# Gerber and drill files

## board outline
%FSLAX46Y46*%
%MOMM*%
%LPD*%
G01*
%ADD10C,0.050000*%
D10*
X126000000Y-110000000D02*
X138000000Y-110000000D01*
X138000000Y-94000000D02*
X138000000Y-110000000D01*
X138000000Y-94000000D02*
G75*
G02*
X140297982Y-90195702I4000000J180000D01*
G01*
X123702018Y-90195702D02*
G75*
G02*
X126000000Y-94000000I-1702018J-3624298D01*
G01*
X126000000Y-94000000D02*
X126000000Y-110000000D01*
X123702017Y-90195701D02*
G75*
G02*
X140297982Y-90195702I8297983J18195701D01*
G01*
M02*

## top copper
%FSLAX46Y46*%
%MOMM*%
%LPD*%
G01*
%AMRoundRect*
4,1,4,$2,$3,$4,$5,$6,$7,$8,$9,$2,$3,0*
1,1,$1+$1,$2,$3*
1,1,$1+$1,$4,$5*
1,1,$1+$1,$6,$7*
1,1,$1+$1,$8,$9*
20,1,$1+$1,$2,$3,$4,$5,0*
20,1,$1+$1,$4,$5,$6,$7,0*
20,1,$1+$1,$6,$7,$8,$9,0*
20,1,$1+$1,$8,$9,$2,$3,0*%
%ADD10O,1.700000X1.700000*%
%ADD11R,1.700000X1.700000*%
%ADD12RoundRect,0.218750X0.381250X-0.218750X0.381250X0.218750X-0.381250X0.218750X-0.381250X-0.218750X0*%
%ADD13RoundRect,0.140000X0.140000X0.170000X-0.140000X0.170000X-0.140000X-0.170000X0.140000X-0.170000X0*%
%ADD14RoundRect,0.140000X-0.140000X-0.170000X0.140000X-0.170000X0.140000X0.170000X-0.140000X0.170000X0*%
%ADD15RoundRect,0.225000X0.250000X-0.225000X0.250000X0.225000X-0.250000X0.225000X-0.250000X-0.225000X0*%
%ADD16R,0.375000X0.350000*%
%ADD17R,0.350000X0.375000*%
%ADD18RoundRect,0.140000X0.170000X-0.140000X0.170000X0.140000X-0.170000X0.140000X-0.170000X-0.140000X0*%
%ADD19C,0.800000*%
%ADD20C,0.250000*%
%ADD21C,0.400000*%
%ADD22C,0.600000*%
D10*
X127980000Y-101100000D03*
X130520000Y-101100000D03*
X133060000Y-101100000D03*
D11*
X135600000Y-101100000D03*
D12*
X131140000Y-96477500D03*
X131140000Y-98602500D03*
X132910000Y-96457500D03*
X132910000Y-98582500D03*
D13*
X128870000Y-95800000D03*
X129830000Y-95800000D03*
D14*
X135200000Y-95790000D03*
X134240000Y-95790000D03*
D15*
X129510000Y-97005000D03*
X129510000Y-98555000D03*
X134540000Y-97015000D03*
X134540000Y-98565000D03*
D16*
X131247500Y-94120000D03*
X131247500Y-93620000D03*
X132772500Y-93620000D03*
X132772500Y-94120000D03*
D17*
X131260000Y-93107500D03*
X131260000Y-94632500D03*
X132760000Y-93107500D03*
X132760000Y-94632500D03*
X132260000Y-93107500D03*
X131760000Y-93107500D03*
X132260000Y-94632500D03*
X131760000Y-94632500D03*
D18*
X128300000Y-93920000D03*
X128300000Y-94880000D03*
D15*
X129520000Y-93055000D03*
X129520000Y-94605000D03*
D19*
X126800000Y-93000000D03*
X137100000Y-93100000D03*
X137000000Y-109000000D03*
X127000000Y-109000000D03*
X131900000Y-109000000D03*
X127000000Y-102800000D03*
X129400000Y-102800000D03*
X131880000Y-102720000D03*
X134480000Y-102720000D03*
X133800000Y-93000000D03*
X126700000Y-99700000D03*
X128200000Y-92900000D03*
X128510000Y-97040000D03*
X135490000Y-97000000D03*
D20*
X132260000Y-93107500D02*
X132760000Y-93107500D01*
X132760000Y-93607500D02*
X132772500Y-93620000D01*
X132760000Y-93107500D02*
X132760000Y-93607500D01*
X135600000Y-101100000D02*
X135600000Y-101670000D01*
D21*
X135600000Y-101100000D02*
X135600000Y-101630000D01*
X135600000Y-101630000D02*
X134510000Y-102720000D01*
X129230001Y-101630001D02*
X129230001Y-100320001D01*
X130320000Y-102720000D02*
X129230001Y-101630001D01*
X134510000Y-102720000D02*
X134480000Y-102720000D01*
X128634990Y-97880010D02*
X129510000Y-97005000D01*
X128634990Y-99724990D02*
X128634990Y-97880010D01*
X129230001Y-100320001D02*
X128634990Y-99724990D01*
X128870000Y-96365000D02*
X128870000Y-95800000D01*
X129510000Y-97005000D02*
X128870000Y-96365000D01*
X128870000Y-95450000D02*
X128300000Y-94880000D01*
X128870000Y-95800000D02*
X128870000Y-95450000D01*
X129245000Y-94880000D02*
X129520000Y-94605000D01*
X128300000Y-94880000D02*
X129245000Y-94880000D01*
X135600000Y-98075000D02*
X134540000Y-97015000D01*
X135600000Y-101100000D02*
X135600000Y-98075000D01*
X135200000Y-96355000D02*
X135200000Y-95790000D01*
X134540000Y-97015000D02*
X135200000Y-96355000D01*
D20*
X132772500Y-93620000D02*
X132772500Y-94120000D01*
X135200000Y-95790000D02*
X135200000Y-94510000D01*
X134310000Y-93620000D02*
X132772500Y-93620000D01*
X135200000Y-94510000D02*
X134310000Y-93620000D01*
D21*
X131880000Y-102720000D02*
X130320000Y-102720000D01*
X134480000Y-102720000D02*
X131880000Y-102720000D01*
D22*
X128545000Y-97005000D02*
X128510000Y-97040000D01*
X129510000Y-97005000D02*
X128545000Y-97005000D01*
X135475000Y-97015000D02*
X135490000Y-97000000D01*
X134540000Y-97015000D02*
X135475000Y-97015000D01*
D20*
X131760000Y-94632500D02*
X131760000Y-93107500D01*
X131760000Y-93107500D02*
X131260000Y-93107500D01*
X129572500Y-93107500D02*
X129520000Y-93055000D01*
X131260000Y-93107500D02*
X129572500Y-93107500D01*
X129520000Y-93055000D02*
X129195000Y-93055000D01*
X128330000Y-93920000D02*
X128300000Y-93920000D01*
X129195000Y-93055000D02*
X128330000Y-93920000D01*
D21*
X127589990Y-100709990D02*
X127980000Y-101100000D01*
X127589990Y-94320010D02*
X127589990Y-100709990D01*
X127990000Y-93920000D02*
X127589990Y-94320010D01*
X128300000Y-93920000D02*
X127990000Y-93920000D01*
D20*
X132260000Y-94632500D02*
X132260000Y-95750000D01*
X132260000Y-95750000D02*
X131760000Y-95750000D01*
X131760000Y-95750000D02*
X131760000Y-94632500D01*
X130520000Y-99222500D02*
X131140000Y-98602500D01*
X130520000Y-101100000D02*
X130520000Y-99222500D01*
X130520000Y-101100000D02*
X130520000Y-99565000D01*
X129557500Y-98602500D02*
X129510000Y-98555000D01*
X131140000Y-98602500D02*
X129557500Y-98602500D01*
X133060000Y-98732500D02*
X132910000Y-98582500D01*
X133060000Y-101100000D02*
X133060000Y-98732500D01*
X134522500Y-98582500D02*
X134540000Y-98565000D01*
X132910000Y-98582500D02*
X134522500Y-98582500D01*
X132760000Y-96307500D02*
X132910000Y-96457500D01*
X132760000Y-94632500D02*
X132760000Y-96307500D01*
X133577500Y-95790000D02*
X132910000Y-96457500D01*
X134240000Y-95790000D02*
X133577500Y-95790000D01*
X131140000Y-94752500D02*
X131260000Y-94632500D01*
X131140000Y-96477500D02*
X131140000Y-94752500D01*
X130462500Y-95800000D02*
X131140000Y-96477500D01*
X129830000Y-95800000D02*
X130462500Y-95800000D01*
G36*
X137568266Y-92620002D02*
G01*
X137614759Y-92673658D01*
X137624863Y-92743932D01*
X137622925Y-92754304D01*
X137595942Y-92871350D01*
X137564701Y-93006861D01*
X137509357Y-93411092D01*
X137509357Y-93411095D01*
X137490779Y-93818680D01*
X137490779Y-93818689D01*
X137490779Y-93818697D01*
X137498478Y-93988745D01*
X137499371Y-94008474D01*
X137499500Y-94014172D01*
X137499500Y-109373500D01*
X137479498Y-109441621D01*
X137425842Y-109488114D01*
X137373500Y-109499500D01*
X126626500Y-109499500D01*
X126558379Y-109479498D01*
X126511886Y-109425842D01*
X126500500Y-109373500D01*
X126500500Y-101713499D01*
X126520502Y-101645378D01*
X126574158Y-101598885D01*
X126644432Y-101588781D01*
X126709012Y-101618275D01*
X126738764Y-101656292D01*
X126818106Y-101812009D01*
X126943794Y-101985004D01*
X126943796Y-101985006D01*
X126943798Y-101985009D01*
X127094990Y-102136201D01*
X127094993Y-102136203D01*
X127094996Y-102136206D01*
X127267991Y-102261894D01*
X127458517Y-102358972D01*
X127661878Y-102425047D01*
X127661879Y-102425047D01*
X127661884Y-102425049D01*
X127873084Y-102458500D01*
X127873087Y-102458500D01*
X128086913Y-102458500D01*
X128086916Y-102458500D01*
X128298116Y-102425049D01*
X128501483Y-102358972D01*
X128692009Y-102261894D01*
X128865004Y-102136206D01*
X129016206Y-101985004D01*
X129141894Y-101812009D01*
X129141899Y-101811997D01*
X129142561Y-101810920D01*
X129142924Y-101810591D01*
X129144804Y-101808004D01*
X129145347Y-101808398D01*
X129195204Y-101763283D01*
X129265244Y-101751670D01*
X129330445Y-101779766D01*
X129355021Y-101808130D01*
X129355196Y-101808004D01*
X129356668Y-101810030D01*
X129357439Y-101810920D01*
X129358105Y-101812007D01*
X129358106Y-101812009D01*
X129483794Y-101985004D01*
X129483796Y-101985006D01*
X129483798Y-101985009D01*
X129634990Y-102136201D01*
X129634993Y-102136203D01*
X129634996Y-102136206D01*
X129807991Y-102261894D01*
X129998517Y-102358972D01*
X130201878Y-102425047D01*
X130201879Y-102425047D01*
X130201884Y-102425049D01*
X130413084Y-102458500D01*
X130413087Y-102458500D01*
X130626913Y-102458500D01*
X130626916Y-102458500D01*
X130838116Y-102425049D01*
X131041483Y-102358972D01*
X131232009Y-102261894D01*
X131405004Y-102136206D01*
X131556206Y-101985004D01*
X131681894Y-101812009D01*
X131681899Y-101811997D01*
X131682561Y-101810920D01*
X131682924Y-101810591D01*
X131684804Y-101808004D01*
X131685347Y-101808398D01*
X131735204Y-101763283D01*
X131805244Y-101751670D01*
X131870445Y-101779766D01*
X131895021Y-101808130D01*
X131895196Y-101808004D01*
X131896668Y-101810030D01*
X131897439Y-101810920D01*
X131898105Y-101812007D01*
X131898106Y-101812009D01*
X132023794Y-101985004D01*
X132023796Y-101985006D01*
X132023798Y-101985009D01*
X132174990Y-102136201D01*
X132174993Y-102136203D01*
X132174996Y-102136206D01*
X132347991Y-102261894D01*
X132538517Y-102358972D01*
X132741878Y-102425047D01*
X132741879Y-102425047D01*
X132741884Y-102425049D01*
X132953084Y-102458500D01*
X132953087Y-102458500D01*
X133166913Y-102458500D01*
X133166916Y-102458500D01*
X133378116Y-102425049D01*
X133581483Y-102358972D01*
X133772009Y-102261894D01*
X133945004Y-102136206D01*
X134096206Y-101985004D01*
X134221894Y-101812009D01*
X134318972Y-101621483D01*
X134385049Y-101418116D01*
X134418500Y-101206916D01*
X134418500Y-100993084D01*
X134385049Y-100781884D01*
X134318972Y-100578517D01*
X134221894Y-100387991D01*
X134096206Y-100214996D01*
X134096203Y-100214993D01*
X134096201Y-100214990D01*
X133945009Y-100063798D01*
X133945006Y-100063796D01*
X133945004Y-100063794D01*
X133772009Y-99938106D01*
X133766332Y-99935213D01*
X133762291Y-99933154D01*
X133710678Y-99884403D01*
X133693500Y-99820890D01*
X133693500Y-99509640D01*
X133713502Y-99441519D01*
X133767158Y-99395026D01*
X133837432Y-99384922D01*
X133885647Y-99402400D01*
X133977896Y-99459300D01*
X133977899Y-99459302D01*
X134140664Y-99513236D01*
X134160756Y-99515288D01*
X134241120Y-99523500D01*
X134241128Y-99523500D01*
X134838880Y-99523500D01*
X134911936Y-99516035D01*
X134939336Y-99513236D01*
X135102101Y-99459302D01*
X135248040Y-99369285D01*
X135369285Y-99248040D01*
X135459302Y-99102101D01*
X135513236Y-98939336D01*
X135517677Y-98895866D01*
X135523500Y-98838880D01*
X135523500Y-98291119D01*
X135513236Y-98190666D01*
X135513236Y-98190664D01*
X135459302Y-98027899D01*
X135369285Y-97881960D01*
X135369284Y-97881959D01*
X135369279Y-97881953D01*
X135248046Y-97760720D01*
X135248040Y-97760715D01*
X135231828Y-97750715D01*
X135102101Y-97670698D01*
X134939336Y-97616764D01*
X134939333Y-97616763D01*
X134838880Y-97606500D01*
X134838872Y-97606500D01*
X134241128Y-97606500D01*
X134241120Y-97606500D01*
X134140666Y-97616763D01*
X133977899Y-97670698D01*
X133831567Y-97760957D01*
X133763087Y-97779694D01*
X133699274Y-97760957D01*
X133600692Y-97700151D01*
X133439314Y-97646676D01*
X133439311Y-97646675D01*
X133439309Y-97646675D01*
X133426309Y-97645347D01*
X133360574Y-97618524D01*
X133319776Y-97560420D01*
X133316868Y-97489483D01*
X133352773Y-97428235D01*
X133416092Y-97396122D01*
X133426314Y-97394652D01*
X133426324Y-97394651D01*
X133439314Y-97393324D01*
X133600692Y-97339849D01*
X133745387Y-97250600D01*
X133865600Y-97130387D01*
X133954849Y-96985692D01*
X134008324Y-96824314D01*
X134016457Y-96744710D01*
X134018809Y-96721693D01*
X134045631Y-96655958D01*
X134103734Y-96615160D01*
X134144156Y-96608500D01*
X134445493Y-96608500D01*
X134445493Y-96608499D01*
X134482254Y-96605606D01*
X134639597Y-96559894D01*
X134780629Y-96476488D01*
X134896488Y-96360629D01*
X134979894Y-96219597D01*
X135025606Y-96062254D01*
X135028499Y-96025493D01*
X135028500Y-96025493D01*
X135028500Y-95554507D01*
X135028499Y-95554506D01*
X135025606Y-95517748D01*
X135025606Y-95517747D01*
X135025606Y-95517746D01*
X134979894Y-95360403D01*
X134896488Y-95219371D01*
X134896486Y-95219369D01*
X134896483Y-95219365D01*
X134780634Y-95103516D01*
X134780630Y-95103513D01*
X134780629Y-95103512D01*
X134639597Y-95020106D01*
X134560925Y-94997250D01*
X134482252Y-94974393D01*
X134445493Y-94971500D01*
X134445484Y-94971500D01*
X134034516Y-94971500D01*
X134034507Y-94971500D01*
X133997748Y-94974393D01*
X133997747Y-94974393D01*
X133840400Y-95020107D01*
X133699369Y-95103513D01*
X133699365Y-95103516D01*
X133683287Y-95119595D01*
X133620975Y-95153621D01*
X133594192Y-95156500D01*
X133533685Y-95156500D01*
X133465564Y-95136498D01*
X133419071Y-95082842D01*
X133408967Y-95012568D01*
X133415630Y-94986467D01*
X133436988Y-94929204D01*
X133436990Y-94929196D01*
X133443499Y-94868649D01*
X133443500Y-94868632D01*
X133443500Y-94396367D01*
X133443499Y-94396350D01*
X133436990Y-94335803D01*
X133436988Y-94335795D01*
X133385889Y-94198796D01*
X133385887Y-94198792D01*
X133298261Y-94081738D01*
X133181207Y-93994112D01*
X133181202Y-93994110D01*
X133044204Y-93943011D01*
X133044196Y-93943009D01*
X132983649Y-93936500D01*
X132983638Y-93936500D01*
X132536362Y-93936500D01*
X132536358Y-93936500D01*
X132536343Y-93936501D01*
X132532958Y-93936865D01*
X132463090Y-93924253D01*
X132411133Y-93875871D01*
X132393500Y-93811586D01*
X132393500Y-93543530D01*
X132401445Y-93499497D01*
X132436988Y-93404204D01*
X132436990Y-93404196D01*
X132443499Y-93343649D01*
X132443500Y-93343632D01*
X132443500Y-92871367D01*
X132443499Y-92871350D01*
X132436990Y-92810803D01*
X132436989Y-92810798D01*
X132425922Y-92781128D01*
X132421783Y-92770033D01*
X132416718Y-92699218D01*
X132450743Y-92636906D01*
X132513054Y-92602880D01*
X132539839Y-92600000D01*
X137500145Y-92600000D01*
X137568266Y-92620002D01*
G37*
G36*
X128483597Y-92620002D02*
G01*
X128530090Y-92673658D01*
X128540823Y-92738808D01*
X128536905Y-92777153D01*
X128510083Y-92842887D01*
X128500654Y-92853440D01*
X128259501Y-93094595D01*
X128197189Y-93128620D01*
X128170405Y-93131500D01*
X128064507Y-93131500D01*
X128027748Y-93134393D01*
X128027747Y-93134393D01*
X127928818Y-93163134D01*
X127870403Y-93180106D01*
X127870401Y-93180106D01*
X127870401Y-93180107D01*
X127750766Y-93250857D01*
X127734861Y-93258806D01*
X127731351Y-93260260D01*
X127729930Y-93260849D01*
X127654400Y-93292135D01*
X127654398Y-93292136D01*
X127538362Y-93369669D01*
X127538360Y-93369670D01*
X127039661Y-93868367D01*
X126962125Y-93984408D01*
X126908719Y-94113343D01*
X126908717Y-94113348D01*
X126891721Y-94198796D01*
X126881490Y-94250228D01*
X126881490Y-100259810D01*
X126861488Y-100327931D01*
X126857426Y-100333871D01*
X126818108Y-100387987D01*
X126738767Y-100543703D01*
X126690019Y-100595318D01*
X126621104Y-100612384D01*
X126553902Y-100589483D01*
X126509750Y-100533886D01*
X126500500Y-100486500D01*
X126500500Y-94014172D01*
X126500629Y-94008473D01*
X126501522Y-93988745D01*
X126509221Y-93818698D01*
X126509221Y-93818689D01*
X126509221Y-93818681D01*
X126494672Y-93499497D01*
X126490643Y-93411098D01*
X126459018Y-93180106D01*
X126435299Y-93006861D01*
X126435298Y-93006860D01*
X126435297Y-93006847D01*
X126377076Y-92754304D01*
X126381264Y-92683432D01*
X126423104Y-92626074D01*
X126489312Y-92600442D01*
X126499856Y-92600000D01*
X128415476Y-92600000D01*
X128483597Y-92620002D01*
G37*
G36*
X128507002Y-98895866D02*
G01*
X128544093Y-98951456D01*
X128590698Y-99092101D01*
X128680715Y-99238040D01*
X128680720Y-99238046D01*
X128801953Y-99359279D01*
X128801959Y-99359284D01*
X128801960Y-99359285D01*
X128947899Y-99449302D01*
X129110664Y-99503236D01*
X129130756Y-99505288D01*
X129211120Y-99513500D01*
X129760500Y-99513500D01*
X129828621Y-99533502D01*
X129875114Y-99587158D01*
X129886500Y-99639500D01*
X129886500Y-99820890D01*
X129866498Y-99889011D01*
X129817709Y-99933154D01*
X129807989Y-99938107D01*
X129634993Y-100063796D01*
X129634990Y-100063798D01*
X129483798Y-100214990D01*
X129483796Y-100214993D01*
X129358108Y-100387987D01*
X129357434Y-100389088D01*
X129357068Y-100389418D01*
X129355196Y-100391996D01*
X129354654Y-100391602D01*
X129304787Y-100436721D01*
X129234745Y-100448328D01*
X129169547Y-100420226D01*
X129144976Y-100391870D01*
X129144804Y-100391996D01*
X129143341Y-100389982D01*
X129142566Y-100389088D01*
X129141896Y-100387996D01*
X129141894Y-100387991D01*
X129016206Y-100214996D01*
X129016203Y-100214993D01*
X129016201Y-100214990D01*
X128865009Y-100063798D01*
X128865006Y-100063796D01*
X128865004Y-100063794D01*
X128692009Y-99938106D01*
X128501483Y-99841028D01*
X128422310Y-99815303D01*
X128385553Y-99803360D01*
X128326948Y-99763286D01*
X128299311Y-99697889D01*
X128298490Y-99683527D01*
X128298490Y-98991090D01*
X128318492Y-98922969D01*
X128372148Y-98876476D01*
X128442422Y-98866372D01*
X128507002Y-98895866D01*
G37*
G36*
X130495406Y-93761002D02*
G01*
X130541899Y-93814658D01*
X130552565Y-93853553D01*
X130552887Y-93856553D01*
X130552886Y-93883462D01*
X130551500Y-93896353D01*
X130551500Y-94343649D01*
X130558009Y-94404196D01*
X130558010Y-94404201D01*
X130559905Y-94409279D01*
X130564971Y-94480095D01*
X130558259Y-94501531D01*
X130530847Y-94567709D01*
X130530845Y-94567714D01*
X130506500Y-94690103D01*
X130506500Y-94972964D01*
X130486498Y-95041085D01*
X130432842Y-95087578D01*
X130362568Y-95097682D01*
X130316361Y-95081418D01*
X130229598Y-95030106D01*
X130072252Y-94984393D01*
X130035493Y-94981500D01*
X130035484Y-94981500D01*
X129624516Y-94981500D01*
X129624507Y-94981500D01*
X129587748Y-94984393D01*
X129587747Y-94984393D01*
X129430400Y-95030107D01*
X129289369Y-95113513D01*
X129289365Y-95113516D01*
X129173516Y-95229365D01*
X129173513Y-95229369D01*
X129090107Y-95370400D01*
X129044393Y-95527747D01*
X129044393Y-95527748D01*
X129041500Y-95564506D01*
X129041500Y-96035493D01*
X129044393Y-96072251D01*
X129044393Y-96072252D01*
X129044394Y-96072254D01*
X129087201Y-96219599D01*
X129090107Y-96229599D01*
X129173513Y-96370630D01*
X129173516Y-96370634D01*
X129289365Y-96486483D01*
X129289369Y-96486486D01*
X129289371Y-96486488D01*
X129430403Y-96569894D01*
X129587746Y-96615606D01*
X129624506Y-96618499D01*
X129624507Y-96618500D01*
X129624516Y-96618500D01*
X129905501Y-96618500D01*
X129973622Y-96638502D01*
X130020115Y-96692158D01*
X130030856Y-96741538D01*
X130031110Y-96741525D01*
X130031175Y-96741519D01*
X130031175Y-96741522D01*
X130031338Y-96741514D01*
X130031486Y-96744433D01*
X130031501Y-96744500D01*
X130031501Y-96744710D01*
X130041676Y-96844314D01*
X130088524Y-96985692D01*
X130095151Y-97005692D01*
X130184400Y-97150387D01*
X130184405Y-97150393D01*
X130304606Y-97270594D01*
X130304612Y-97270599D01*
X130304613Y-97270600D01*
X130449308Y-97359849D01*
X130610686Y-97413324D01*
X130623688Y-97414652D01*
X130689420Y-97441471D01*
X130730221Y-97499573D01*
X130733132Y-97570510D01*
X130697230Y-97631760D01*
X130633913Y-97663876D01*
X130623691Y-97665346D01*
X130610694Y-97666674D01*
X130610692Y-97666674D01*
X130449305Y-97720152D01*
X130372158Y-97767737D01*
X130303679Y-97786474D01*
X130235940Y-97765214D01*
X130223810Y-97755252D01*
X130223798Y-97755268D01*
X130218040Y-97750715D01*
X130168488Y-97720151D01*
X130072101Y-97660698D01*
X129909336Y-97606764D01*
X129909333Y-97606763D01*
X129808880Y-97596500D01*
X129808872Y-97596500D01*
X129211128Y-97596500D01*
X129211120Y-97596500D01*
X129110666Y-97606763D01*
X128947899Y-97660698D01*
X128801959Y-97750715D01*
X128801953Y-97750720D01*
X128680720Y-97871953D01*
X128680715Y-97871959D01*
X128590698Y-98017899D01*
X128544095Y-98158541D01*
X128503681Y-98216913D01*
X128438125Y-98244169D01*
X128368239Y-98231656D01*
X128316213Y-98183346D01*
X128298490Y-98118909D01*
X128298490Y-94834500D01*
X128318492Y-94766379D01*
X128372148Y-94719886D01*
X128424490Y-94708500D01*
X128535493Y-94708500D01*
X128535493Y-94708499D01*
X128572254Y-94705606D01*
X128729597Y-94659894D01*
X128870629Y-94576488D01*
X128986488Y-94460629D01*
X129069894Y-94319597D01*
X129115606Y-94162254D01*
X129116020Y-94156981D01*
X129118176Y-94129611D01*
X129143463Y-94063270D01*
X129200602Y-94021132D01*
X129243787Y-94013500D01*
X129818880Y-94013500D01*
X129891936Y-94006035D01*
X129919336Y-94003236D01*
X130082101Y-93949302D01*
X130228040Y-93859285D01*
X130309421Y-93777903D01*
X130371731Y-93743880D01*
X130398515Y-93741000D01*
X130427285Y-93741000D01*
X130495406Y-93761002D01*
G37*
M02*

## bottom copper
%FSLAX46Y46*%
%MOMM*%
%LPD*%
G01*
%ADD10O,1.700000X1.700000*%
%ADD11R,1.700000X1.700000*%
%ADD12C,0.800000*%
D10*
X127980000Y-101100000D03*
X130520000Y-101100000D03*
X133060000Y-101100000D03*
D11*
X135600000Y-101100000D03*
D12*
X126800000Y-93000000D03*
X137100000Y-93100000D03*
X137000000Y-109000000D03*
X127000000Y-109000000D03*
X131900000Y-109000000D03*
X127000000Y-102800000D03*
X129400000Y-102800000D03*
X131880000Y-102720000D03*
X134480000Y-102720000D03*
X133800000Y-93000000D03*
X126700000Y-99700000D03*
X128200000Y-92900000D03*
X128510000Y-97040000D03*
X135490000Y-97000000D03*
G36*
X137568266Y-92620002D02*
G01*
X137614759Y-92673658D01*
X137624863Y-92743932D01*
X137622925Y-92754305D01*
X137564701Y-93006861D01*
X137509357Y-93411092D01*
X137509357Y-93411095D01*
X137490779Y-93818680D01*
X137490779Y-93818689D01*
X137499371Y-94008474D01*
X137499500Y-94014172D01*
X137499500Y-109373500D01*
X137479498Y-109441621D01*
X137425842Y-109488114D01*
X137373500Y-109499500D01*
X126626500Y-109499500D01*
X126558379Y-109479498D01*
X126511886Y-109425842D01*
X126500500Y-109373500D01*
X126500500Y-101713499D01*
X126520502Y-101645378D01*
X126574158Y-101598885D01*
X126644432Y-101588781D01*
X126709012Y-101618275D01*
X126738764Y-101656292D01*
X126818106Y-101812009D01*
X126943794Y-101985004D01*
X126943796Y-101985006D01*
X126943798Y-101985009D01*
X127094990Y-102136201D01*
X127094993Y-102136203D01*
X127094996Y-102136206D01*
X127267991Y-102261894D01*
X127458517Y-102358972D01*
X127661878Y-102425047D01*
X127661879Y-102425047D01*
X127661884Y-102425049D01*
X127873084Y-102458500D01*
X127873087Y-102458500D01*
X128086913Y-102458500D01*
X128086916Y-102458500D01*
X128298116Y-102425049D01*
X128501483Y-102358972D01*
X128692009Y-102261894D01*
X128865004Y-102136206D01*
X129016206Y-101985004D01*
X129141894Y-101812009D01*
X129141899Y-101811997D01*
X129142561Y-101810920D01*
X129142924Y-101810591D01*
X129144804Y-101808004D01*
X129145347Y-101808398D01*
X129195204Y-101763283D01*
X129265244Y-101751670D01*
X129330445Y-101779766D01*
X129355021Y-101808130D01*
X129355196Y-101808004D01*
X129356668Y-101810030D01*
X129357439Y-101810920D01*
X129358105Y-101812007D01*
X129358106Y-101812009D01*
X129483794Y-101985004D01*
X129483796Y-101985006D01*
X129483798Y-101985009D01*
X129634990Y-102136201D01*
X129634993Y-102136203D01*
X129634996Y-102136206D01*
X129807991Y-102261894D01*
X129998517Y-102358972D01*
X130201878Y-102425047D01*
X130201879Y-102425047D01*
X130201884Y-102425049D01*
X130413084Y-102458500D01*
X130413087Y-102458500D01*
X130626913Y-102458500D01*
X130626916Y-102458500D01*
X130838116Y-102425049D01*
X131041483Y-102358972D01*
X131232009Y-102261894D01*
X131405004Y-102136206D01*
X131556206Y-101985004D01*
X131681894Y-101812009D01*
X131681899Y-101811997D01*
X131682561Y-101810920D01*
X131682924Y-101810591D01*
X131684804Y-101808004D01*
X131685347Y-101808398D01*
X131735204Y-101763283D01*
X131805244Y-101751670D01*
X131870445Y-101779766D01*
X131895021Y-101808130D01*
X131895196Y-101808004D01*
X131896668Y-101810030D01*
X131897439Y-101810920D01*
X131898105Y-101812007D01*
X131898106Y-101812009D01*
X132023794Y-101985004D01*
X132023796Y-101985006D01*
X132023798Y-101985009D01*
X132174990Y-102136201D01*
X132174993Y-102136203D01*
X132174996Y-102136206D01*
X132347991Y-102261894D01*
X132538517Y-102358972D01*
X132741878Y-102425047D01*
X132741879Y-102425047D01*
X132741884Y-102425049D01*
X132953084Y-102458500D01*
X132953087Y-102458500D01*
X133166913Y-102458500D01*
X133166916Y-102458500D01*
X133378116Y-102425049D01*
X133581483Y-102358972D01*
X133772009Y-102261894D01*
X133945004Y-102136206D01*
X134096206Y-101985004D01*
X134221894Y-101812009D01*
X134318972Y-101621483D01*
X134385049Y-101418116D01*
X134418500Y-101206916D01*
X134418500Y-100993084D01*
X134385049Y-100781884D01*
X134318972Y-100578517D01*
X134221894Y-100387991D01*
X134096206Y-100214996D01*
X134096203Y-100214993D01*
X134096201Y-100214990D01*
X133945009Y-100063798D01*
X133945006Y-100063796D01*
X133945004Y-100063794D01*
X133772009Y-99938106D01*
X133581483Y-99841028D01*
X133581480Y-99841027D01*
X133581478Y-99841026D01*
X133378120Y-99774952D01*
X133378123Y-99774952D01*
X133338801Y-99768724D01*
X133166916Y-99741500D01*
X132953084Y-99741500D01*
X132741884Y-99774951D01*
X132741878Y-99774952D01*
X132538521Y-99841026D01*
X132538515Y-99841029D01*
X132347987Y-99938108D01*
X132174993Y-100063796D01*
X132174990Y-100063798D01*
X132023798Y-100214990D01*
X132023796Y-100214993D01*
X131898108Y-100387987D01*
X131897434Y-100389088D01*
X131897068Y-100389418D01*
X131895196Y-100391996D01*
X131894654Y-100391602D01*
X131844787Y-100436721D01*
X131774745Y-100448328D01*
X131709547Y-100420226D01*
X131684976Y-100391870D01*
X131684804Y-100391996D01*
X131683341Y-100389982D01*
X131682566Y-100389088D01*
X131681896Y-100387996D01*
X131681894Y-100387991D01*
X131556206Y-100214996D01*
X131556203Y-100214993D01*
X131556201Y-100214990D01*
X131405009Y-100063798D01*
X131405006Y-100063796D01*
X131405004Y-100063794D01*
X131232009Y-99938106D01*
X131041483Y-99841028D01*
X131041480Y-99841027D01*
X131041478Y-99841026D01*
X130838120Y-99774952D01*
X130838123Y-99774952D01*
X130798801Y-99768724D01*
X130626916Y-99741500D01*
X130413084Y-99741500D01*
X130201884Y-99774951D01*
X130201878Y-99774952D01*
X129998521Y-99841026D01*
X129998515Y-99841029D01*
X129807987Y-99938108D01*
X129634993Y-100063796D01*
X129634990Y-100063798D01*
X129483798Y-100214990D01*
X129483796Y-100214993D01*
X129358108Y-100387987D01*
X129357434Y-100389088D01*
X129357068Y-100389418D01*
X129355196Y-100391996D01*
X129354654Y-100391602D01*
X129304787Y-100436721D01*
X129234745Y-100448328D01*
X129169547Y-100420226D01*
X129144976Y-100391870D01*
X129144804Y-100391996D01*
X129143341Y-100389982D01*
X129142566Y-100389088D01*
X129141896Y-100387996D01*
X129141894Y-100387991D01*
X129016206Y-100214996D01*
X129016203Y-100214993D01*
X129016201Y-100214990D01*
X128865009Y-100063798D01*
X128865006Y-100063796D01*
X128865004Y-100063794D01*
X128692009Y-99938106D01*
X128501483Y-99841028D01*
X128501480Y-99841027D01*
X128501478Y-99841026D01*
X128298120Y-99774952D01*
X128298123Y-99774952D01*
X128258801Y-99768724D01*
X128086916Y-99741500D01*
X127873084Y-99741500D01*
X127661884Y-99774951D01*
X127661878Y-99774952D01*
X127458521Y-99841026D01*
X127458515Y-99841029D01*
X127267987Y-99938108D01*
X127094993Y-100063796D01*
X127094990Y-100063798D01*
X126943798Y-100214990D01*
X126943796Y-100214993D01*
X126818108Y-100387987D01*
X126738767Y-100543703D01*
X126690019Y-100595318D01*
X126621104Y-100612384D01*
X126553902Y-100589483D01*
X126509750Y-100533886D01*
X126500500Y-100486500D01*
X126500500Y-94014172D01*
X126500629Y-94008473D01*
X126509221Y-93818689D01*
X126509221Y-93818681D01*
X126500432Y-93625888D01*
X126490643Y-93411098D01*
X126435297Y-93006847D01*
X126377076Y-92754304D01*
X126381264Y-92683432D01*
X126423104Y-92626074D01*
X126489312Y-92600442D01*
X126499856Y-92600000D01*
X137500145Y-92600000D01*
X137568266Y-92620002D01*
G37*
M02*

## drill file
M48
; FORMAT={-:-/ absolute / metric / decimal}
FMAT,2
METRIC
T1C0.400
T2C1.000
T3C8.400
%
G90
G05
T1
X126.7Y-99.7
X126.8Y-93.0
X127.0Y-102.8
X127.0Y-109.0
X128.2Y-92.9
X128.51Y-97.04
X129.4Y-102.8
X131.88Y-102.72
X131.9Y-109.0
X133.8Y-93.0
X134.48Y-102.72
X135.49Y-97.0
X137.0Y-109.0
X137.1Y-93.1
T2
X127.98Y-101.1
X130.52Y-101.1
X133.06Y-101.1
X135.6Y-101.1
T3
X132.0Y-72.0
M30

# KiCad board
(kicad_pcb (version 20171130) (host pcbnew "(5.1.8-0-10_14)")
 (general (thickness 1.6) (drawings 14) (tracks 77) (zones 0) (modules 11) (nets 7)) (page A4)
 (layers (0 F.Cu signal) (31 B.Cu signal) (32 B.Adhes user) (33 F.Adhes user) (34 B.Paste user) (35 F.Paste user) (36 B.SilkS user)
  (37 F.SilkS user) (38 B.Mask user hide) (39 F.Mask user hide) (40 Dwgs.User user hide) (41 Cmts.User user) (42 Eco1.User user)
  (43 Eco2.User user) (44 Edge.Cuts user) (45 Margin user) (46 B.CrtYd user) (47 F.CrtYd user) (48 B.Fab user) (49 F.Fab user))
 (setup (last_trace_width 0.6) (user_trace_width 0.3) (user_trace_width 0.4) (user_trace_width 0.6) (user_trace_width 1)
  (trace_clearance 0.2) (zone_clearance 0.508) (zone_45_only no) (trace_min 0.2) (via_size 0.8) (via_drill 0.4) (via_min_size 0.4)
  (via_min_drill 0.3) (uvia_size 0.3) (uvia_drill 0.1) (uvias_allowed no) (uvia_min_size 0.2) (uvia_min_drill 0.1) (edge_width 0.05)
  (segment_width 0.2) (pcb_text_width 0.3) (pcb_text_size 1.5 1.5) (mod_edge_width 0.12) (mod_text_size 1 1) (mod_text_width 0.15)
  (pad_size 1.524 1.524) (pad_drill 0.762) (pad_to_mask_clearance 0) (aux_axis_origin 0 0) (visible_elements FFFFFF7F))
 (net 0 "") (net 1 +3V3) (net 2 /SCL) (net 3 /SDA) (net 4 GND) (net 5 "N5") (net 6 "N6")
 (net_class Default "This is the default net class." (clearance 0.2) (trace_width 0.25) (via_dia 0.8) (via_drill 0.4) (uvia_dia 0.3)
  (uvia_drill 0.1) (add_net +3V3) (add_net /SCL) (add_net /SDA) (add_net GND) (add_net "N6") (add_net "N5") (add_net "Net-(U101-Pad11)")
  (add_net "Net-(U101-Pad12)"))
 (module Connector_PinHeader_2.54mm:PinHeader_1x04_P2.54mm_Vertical (layer F.Cu) (at 135.6 101.1 270)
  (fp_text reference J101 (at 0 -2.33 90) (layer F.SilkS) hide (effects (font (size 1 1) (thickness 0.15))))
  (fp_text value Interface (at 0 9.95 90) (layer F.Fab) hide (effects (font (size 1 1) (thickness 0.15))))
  (pad 4 thru_hole oval (at 0 7.62 270) (size 1.7 1.7) (drill 1) (layers *.Cu *.Mask) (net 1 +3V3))
  (pad 3 thru_hole oval (at 0 5.08 270) (size 1.7 1.7) (drill 1) (layers *.Cu *.Mask) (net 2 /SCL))
  (pad 2 thru_hole oval (at 0 2.54 270) (size 1.7 1.7) (drill 1) (layers *.Cu *.Mask) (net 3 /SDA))
  (pad 1 thru_hole rect (at 0 0 270) (size 1.7 1.7) (drill 1) (layers *.Cu *.Mask) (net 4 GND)))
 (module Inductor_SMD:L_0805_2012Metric (layer F.Cu) (at 131.14 97.54 90)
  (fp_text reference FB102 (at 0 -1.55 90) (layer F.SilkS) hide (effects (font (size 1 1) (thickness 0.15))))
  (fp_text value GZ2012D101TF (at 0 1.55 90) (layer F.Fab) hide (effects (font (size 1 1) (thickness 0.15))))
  (pad 2 smd roundrect (at 1.0625 0 90) (size 0.875 1.2) (layers F.Cu F.Paste F.Mask) (roundrect_rratio 0.25) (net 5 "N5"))
  (pad 1 smd roundrect (at -1.0625 0 90) (size 0.875 1.2) (layers F.Cu F.Paste F.Mask) (roundrect_rratio 0.25) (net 2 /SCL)))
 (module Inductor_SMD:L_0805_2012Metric (layer F.Cu) (at 132.91 97.52 90)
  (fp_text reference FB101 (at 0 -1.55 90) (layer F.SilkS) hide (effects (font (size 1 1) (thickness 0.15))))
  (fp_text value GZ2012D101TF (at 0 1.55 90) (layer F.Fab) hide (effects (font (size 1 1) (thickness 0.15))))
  (pad 2 smd roundrect (at 1.0625 0 90) (size 0.875 1.2) (layers F.Cu F.Paste F.Mask) (roundrect_rratio 0.25) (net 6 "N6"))
  (pad 1 smd roundrect (at -1.0625 0 90) (size 0.875 1.2) (layers F.Cu F.Paste F.Mask) (roundrect_rratio 0.25) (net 3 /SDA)))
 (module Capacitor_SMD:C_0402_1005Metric (layer F.Cu) (at 129.35 95.8 180)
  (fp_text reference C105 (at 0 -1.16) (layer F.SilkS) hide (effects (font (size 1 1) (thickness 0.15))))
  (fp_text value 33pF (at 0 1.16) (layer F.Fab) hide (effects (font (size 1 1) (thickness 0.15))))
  (pad 2 smd roundrect (at 0.48 0 180) (size 0.56 0.62) (layers F.Cu F.Paste F.Mask) (roundrect_rratio 0.25) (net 4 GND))
  (pad 1 smd roundrect (at -0.48 0 180) (size 0.56 0.62) (layers F.Cu F.Paste F.Mask) (roundrect_rratio 0.25) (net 5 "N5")))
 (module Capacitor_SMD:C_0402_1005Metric (layer F.Cu) (at 134.72 95.79)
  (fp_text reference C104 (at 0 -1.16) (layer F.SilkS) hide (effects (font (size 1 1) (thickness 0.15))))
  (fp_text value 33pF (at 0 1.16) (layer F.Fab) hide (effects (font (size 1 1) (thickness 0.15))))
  (pad 2 smd roundrect (at 0.48 0) (size 0.56 0.62) (layers F.Cu F.Paste F.Mask) (roundrect_rratio 0.25) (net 4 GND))
  (pad 1 smd roundrect (at -0.48 0) (size 0.56 0.62) (layers F.Cu F.Paste F.Mask) (roundrect_rratio 0.25) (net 6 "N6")))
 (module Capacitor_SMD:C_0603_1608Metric (layer F.Cu) (at 129.51 97.78 90)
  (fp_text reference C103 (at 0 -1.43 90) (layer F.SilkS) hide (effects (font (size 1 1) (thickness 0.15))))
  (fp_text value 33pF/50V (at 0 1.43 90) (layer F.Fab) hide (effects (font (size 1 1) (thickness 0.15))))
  (pad 2 smd roundrect (at 0.775 0 90) (size 0.9 0.95) (layers F.Cu F.Paste F.Mask) (roundrect_rratio 0.25) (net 4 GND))
  (pad 1 smd roundrect (at -0.775 0 90) (size 0.9 0.95) (layers F.Cu F.Paste F.Mask) (roundrect_rratio 0.25) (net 2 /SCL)))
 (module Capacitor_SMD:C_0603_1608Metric (layer F.Cu) (at 134.54 97.79 90)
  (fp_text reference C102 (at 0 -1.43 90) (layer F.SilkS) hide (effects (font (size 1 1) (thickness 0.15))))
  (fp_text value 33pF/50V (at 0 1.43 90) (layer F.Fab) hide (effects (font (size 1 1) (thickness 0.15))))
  (pad 2 smd roundrect (at 0.775 0 90) (size 0.9 0.95) (layers F.Cu F.Paste F.Mask) (roundrect_rratio 0.25) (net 4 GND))
  (pad 1 smd roundrect (at -0.775 0 90) (size 0.9 0.95) (layers F.Cu F.Paste F.Mask) (roundrect_rratio 0.25) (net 3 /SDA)))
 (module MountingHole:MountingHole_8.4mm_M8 (layer F.Cu) (at 132 72)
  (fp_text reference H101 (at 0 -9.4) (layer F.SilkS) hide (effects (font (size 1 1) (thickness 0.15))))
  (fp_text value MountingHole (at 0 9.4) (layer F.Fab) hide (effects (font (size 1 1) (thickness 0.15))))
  (pad 1 np_thru_hole circle (at 0 0) (size 8.4 8.4) (drill 8.4) (layers *.Cu *.Mask)))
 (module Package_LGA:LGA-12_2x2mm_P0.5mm (layer F.Cu) (at 132.01 93.87 90)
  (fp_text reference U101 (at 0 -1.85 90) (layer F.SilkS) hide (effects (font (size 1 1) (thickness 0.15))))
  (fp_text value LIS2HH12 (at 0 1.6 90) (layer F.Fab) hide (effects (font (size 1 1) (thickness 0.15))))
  (pad 12 smd rect (at -0.25 -0.7625 180) (size 0.375 0.35) (layers F.Cu F.Paste F.Mask))
  (pad 11 smd rect (at 0.25 -0.7625 180) (size 0.375 0.35) (layers F.Cu F.Paste F.Mask))
  (pad 6 smd rect (at 0.25 0.7625 180) (size 0.375 0.35) (layers F.Cu F.Paste F.Mask) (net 4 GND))
  (pad 5 smd rect (at -0.25 0.7625 180) (size 0.375 0.35) (layers F.Cu F.Paste F.Mask) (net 4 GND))
  (pad 10 smd rect (at 0.7625 -0.75 90) (size 0.375 0.35) (layers F.Cu F.Paste F.Mask) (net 1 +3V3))
  (pad 1 smd rect (at -0.7625 -0.75 90) (size 0.375 0.35) (layers F.Cu F.Paste F.Mask) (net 5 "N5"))
  (pad 7 smd rect (at 0.7625 0.75 90) (size 0.375 0.35) (layers F.Cu F.Paste F.Mask) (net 4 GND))
  (pad 4 smd rect (at -0.7625 0.75 90) (size 0.375 0.35) (layers F.Cu F.Paste F.Mask) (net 6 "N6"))
  (pad 8 smd rect (at 0.7625 0.25 90) (size 0.375 0.35) (layers F.Cu F.Paste F.Mask) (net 4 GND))
  (pad 9 smd rect (at 0.7625 -0.25 90) (size 0.375 0.35) (layers F.Cu F.Paste F.Mask) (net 1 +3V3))
  (pad 3 smd rect (at -0.7625 0.25 90) (size 0.375 0.35) (layers F.Cu F.Paste F.Mask) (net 1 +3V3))
  (pad 2 smd rect (at -0.7625 -0.25 90) (size 0.375 0.35) (layers F.Cu F.Paste F.Mask) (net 1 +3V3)))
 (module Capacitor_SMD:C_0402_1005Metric (layer F.Cu) (at 128.3 94.4 90)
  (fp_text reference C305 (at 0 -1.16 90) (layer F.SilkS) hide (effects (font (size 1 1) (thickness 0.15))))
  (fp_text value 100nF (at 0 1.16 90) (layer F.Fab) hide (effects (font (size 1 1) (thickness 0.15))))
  (pad 2 smd roundrect (at 0.48 0 90) (size 0.56 0.62) (layers F.Cu F.Paste F.Mask) (roundrect_rratio 0.25) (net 1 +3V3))
  (pad 1 smd roundrect (at -0.48 0 90) (size 0.56 0.62) (layers F.Cu F.Paste F.Mask) (roundrect_rratio 0.25) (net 4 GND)))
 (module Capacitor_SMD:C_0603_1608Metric (layer F.Cu) (at 129.52 93.83 90)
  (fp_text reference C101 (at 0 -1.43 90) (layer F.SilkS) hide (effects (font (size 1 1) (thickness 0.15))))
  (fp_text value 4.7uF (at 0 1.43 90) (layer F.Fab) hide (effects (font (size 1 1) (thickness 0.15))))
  (pad 2 smd roundrect (at 0.775 0 90) (size 0.9 0.95) (layers F.Cu F.Paste F.Mask) (roundrect_rratio 0.25) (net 1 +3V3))
  (pad 1 smd roundrect (at -0.775 0 90) (size 0.9 0.95) (layers F.Cu F.Paste F.Mask) (roundrect_rratio 0.25) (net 4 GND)))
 (gr_line (start 126 110) (end 138 110) (layer Edge.Cuts) (width 0.05))
 (gr_line (start 138 94) (end 138 110) (layer Edge.Cuts) (width 0.05))
 (gr_arc (start 142 93.82) (end 138 94) (angle 67.4211994) (layer Edge.Cuts) (width 0.05))
 (gr_arc (start 122 93.82) (end 126 94) (angle -67.4211994) (layer Edge.Cuts) (width 0.05))
 (gr_line (start 126 94) (end 126 110) (layer Edge.Cuts) (width 0.05))
 (gr_arc (start 132 72) (end 140.297982 90.195702) (angle -310.9701567) (layer Edge.Cuts) (width 0.05))
 (segment (start 132.26 93.1075) (end 132.76 93.1075) (width 0.25) (layer F.Cu) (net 4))
 (segment (start 132.76 93.6075) (end 132.7725 93.62) (width 0.25) (layer F.Cu) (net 4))
 (segment (start 132.76 93.1075) (end 132.76 93.6075) (width 0.25) (layer F.Cu) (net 4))
 (segment (start 135.6 101.1) (end 135.6 101.67) (width 0.25) (layer F.Cu) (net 4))
 (segment (start 135.6 101.1) (end 135.6 101.63) (width 0.4) (layer F.Cu) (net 4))
 (segment (start 135.6 101.63) (end 134.51 102.72) (width 0.4) (layer F.Cu) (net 4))
 (segment (start 129.230001 101.630001) (end 129.230001 100.320001) (width 0.4) (layer F.Cu) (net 4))
 (segment (start 130.32 102.72) (end 129.230001 101.630001) (width 0.4) (layer F.Cu) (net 4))
 (segment (start 134.51 102.72) (end 134.48 102.72) (width 0.4) (layer F.Cu) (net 4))
 (segment (start 128.63499 97.88001) (end 129.51 97.005) (width 0.4) (layer F.Cu) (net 4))
 (segment (start 128.63499 99.72499) (end 128.63499 97.88001) (width 0.4) (layer F.Cu) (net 4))
 (segment (start 129.230001 100.320001) (end 128.63499 99.72499) (width 0.4) (layer F.Cu) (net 4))
 (segment (start 128.87 96.365) (end 128.87 95.8) (width 0.4) (layer F.Cu) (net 4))
 (segment (start 129.51 97.005) (end 128.87 96.365) (width 0.4) (layer F.Cu) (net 4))
 (segment (start 128.87 95.45) (end 128.3 94.88) (width 0.4) (layer F.Cu) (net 4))
 (segment (start 128.87 95.8) (end 128.87 95.45) (width 0.4) (layer F.Cu) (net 4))
 (segment (start 129.245 94.88) (end 129.52 94.605) (width 0.4) (layer F.Cu) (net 4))
 (segment (start 128.3 94.88) (end 129.245 94.88) (width 0.4) (layer F.Cu) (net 4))
 (segment (start 135.6 98.075) (end 134.54 97.015) (width 0.4) (layer F.Cu) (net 4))
 (segment (start 135.6 101.1) (end 135.6 98.075) (width 0.4) (layer F.Cu) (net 4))
 (segment (start 135.2 96.355) (end 135.2 95.79) (width 0.4) (layer F.Cu) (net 4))
 (segment (start 134.54 97.015) (end 135.2 96.355) (width 0.4) (layer F.Cu) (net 4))
 (segment (start 132.7725 93.62) (end 132.7725 94.12) (width 0.25) (layer F.Cu) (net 4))
 (segment (start 135.2 95.79) (end 135.2 94.51) (width 0.25) (layer F.Cu) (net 4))
 (segment (start 134.31 93.62) (end 132.7725 93.62) (width 0.25) (layer F.Cu) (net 4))
 (segment (start 135.2 94.51) (end 134.31 93.62) (width 0.25) (layer F.Cu) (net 4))
 (via (at 126.8 93) (size 0.8) (drill 0.4) (layers F.Cu B.Cu) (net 4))
 (via (at 137.1 93.1) (size 0.8) (drill 0.4) (layers F.Cu B.Cu) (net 4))
 (via (at 137 109) (size 0.8) (drill 0.4) (layers F.Cu B.Cu) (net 4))
 (via (at 127 109) (size 0.8) (drill 0.4) (layers F.Cu B.Cu) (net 4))
 (via (at 131.9 109) (size 0.8) (drill 0.4) (layers F.Cu B.Cu) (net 4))
 (via (at 127 102.8) (size 0.8) (drill 0.4) (layers F.Cu B.Cu) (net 4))
 (via (at 129.4 102.8) (size 0.8) (drill 0.4) (layers F.Cu B.Cu) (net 4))
 (segment (start 131.88 102.72) (end 130.32 102.72) (width 0.4) (layer F.Cu) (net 4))
 (via (at 131.88 102.72) (size 0.8) (drill 0.4) (layers F.Cu B.Cu) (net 4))
 (segment (start 134.48 102.72) (end 131.88 102.72) (width 0.4) (layer F.Cu) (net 4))
 (via (at 134.48 102.72) (size 0.8) (drill 0.4) (layers F.Cu B.Cu) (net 4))
 (via (at 133.8 93) (size 0.8) (drill 0.4) (layers F.Cu B.Cu) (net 4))
 (via (at 126.7 99.7) (size 0.8) (drill 0.4) (layers F.Cu B.Cu) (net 4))
 (via (at 128.2 92.9) (size 0.8) (drill 0.4) (layers F.Cu B.Cu) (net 4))
 (via (at 128.51 97.04) (size 0.8) (drill 0.4) (layers F.Cu B.Cu) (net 4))
 (segment (start 128.545 97.005) (end 128.51 97.04) (width 0.6) (layer F.Cu) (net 4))
 (segment (start 129.51 97.005) (end 128.545 97.005) (width 0.6) (layer F.Cu) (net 4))
 (via (at 135.49 97) (size 0.8) (drill 0.4) (layers F.Cu B.Cu) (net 4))
 (segment (start 135.475 97.015) (end 135.49 97) (width 0.6) (layer F.Cu) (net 4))
 (segment (start 134.54 97.015) (end 135.475 97.015) (width 0.6) (layer F.Cu) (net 4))
 (segment (start 131.76 94.6325) (end 131.76 93.1075) (width 0.25) (layer F.Cu) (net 1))
 (segment (start 131.76 93.1075) (end 131.26 93.1075) (width 0.25) (layer F.Cu) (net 1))
 (segment (start 129.5725 93.1075) (end 129.52 93.055) (width 0.25) (layer F.Cu) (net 1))
 (segment (start 131.26 93.1075) (end 129.5725 93.1075) (width 0.25) (layer F.Cu) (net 1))
 (segment (start 129.52 93.055) (end 129.195 93.055) (width 0.25) (layer F.Cu) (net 1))
 (segment (start 128.33 93.92) (end 128.3 93.92) (width 0.25) (layer F.Cu) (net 1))
 (segment (start 129.195 93.055) (end 128.33 93.92) (width 0.25) (layer F.Cu) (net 1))
 (segment (start 127.58999 100.70999) (end 127.98 101.1) (width 0.4) (layer F.Cu) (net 1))
 (segment (start 127.58999 94.32001) (end 127.58999 100.70999) (width 0.4) (layer F.Cu) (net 1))
 (segment (start 127.99 93.92) (end 127.58999 94.32001) (width 0.4) (layer F.Cu) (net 1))
 (segment (start 128.3 93.92) (end 127.99 93.92) (width 0.4) (layer F.Cu) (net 1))
 (segment (start 132.26 94.6325) (end 132.26 95.75) (width 0.25) (layer F.Cu) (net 1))
 (segment (start 132.26 95.75) (end 131.76 95.75) (width 0.25) (layer F.Cu) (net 1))
 (segment (start 131.76 95.75) (end 131.76 94.6325) (width 0.25) (layer F.Cu) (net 1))
 (segment (start 130.52 99.2225) (end 131.14 98.6025) (width 0.25) (layer F.Cu) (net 2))
 (segment (start 130.52 101.1) (end 130.52 99.2225) (width 0.25) (layer F.Cu) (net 2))
 (segment (start 130.52 101.1) (end 130.52 99.565) (width 0.25) (layer F.Cu) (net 2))
 (segment (start 129.5575 98.6025) (end 129.51 98.555) (width 0.25) (layer F.Cu) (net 2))
 (segment (start 131.14 98.6025) (end 129.5575 98.6025) (width 0.25) (layer F.Cu) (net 2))
 (segment (start 133.06 98.7325) (end 132.91 98.5825) (width 0.25) (layer F.Cu) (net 3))
 (segment (start 133.06 101.1) (end 133.06 98.7325) (width 0.25) (layer F.Cu) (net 3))
 (segment (start 134.5225 98.5825) (end 134.54 98.565) (width 0.25) (layer F.Cu) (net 3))
 (segment (start 132.91 98.5825) (end 134.5225 98.5825) (width 0.25) (layer F.Cu) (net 3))
 (segment (start 132.76 96.3075) (end 132.91 96.4575) (width 0.25) (layer F.Cu) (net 6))
 (segment (start 132.76 94.6325) (end 132.76 96.3075) (width 0.25) (layer F.Cu) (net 6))
 (segment (start 133.5775 95.79) (end 132.91 96.4575) (width 0.25) (layer F.Cu) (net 6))
 (segment (start 134.24 95.79) (end 133.5775 95.79) (width 0.25) (layer F.Cu) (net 6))
 (segment (start 131.14 94.7525) (end 131.26 94.6325) (width 0.25) (layer F.Cu) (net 5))
 (segment (start 131.14 96.4775) (end 131.14 94.7525) (width 0.25) (layer F.Cu) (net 5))
 (segment (start 130.4625 95.8) (end 131.14 96.4775) (width 0.25) (layer F.Cu) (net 5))
 (segment (start 129.83 95.8) (end 130.4625 95.8) (width 0.25) (layer F.Cu) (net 5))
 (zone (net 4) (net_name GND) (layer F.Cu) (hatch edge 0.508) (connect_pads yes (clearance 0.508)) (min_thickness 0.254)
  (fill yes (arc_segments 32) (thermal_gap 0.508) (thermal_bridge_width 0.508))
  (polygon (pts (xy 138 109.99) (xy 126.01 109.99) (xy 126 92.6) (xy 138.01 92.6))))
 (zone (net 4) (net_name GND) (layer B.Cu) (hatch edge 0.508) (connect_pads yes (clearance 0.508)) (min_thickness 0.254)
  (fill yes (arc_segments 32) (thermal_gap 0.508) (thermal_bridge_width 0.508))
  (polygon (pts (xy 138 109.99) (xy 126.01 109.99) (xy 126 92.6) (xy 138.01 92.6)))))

